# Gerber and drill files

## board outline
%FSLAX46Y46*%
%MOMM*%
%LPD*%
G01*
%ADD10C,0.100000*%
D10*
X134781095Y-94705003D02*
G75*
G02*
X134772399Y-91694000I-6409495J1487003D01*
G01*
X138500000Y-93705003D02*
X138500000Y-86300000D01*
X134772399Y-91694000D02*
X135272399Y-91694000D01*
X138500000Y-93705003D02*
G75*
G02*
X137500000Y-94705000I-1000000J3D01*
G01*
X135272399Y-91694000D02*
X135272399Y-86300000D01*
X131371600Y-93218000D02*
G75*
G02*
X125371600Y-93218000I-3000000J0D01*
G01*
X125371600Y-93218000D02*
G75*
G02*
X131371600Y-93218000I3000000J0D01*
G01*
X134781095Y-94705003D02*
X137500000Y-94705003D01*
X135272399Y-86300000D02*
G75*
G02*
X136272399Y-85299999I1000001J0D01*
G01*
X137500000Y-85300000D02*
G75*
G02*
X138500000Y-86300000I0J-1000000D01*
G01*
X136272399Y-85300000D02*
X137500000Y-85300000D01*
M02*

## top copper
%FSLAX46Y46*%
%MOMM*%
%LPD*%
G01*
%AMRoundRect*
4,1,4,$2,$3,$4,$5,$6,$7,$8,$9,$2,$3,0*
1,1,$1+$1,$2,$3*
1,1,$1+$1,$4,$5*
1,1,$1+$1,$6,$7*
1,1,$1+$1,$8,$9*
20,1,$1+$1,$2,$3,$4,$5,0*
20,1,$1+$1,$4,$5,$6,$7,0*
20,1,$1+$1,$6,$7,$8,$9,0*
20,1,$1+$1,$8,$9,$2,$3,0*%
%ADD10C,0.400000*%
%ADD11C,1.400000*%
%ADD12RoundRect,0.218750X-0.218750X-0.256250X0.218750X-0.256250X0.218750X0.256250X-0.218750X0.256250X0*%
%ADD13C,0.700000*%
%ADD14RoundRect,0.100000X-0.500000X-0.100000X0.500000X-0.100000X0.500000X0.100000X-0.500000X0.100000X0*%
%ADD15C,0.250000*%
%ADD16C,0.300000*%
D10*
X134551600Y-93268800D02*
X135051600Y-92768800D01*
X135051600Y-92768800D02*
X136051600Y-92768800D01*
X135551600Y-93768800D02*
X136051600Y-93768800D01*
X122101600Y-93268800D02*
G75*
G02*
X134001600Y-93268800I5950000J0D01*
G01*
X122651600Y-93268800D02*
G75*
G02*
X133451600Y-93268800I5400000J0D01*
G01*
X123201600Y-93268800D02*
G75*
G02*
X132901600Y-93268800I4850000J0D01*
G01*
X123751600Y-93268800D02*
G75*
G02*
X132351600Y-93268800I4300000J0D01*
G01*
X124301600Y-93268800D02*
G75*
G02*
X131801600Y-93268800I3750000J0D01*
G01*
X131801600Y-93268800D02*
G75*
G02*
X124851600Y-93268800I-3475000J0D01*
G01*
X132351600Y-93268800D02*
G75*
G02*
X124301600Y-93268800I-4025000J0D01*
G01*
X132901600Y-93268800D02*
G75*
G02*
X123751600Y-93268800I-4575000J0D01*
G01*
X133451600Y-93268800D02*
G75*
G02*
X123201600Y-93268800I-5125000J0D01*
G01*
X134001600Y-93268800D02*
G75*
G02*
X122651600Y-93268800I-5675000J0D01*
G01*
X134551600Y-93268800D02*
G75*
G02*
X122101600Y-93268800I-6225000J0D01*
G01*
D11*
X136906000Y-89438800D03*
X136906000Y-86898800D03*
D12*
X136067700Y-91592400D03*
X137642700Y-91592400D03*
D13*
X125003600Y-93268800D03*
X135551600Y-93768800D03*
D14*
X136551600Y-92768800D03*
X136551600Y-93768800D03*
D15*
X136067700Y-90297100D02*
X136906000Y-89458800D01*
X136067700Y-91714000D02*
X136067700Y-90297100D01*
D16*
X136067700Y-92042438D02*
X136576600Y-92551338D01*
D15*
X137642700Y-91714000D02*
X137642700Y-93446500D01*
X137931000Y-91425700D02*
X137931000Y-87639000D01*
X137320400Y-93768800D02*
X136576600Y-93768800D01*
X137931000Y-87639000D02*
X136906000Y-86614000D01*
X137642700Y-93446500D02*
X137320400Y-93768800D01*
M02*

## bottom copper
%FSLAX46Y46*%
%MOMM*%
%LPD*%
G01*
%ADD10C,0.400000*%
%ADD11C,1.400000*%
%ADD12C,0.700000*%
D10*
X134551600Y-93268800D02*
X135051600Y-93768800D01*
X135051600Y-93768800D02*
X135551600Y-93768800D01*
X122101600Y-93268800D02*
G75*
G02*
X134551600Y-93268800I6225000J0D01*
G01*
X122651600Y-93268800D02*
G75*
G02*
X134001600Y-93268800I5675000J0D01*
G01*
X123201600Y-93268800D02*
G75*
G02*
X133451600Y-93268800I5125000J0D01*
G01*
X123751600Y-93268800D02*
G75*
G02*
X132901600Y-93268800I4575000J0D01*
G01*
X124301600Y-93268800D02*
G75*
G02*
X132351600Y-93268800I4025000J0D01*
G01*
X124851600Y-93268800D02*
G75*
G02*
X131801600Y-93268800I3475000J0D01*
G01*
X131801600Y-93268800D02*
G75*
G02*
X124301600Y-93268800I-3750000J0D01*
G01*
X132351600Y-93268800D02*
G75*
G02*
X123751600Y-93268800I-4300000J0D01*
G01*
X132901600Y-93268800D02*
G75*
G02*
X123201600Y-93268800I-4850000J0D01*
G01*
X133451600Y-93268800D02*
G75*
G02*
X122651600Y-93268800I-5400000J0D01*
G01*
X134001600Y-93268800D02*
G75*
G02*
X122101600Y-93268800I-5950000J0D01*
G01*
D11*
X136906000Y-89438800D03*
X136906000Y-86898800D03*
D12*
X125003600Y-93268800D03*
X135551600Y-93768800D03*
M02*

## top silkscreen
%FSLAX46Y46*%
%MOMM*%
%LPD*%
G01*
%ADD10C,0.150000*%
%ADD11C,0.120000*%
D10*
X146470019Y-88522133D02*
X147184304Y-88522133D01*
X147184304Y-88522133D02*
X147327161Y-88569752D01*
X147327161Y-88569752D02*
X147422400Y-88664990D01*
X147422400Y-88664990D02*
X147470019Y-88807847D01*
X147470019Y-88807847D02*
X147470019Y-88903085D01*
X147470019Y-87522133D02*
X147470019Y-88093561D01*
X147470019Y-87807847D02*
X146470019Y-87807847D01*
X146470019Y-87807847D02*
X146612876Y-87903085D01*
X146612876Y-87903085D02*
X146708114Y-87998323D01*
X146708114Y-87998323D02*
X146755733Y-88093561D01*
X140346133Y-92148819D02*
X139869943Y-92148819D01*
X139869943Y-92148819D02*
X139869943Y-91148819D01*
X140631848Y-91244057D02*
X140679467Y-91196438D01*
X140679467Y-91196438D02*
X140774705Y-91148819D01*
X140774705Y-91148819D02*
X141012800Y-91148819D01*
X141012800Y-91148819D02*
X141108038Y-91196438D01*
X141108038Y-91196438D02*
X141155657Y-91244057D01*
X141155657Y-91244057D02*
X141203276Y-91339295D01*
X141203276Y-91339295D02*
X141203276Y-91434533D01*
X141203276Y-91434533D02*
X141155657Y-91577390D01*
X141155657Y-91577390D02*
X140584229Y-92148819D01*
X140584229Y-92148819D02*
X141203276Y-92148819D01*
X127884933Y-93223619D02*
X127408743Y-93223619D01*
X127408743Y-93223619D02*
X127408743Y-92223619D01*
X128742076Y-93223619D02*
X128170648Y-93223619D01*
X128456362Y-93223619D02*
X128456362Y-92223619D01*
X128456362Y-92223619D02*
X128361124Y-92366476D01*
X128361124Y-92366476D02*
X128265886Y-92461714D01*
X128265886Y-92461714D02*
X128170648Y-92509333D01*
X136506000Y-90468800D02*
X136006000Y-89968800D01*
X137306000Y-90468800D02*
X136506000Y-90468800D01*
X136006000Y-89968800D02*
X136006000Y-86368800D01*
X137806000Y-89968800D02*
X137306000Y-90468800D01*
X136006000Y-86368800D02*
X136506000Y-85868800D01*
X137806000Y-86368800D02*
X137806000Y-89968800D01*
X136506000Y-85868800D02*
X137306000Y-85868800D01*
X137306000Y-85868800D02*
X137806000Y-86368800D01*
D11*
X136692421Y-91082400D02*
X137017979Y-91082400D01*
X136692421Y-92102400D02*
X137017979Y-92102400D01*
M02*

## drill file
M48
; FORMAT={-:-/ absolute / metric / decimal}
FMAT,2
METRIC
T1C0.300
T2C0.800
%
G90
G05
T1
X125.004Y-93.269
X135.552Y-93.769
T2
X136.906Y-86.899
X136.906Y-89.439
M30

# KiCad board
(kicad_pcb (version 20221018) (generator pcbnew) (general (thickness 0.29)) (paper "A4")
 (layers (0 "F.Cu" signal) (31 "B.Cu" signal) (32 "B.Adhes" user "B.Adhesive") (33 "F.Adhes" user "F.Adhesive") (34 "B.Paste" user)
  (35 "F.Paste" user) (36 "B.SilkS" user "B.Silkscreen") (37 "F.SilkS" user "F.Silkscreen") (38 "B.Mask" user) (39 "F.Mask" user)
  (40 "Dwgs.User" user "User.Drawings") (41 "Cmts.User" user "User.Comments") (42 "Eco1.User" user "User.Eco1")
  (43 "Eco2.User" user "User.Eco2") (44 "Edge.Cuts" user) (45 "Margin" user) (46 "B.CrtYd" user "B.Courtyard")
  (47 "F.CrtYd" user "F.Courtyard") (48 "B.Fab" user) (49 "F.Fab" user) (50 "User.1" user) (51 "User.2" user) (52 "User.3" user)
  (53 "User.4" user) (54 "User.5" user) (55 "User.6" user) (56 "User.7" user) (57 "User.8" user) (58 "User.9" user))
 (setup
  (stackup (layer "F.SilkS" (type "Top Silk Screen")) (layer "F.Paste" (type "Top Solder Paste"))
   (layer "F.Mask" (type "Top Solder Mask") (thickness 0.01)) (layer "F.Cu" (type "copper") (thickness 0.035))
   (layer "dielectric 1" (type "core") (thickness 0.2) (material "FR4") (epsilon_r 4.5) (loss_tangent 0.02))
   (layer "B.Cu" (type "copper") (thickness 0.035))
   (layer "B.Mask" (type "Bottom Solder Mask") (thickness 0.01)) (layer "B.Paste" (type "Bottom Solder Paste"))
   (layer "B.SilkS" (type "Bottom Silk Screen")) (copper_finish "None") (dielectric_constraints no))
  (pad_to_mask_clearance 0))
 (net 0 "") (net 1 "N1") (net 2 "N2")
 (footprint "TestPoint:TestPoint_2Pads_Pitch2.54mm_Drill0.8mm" (layer "F.Cu") (at 136.906 89.4388 90)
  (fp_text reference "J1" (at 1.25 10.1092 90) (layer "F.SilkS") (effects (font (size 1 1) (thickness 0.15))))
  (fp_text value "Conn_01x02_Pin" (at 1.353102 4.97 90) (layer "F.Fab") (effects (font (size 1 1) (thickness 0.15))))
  (fp_line (start -1.03 -0.4) (end -0.53 -0.9) (stroke (width 0.15) (type solid)) (layer "F.SilkS"))
  (fp_line (start -1.03 0.4) (end -1.03 -0.4) (stroke (width 0.15) (type solid)) (layer "F.SilkS"))
  (fp_line (start -0.53 -0.9) (end 3.07 -0.9) (stroke (width 0.15) (type solid)) (layer "F.SilkS"))
  (fp_line (start -0.53 0.9) (end -1.03 0.4) (stroke (width 0.15) (type solid)) (layer "F.SilkS"))
  (fp_line (start 3.07 -0.9) (end 3.57 -0.4) (stroke (width 0.15) (type solid)) (layer "F.SilkS"))
  (fp_line (start 3.07 0.9) (end -0.53 0.9) (stroke (width 0.15) (type solid)) (layer "F.SilkS"))
  (fp_line (start 3.57 -0.4) (end 3.57 0.4) (stroke (width 0.15) (type solid)) (layer "F.SilkS"))
  (fp_line (start 3.57 0.4) (end 3.07 0.9) (stroke (width 0.15) (type solid)) (layer "F.SilkS"))
  (pad "1" thru_hole circle (at 0 0 90) (size 1.4 1.4) (drill 0.8) (layers "*.Cu" "*.Mask") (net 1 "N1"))
  (pad "2" thru_hole circle (at 2.54 0 90) (size 1.4 1.4) (drill 0.8) (layers "*.Cu" "*.Mask") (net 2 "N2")))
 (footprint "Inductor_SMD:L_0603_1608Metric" (layer "F.Cu") (at 136.8552 91.5924)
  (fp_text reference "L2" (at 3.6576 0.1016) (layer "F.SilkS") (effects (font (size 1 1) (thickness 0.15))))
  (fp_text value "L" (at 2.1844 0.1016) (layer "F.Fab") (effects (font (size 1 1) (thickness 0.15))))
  (fp_line (start -0.162779 -0.51) (end 0.162779 -0.51) (stroke (width 0.12) (type solid)) (layer "F.SilkS"))
  (fp_line (start -0.162779 0.51) (end 0.162779 0.51) (stroke (width 0.12) (type solid)) (layer "F.SilkS"))
  (pad "1" smd roundrect (at -0.7875 0) (size 0.875 0.95) (layers "F.Cu" "F.Paste" "F.Mask") (roundrect_rratio 0.25) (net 1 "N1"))
  (pad "2" smd roundrect (at 0.7875 0) (size 0.875 0.95) (layers "F.Cu" "F.Paste" "F.Mask") (roundrect_rratio 0.25) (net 2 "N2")))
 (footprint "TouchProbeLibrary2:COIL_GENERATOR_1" (layer "F.Cu") (at 128.3716 93.2688)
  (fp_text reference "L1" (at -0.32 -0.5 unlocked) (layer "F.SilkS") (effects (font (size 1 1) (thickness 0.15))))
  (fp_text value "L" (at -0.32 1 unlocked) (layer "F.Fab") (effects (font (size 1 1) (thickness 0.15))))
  (fp_line (start 6.18 0) (end 6.68 -0.5) (stroke (width 0.4) (type solid)) (layer "F.Cu"))
  (fp_line (start 6.68 -0.5) (end 7.68 -0.5) (stroke (width 0.4) (type solid)) (layer "F.Cu"))
  (fp_line (start 7.18 0.5) (end 7.68 0.5) (stroke (width 0.4) (type solid)) (layer "F.Cu"))
  (fp_arc (start -6.27 0) (mid -0.32 -5.95) (end 5.63 0) (stroke (width 0.4) (type solid)) (layer "F.Cu"))
  (fp_arc (start -5.72 0) (mid -0.32 -5.4) (end 5.08 0) (stroke (width 0.4) (type solid)) (layer "F.Cu"))
  (fp_arc (start -5.17 0) (mid -0.32 -4.85) (end 4.53 0) (stroke (width 0.4) (type solid)) (layer "F.Cu"))
  (fp_arc (start -4.62 0) (mid -0.32 -4.3) (end 3.98 0) (stroke (width 0.4) (type solid)) (layer "F.Cu"))
  (fp_arc (start -4.07 0) (mid -0.32 -3.75) (end 3.43 0) (stroke (width 0.4) (type solid)) (layer "F.Cu"))
  (fp_arc (start 3.43 0) (mid -0.045 3.475) (end -3.52 0) (stroke (width 0.4) (type solid)) (layer "F.Cu"))
  (fp_arc (start 3.98 0) (mid -0.045 4.025) (end -4.07 0) (stroke (width 0.4) (type solid)) (layer "F.Cu"))
  (fp_arc (start 4.53 0) (mid -0.045 4.575) (end -4.62 0) (stroke (width 0.4) (type solid)) (layer "F.Cu"))
  (fp_arc (start 5.08 0) (mid -0.045 5.125) (end -5.17 0) (stroke (width 0.4) (type solid)) (layer "F.Cu"))
  (fp_arc (start 5.63 0) (mid -0.045 5.675) (end -5.72 0) (stroke (width 0.4) (type solid)) (layer "F.Cu"))
  (fp_arc (start 6.18 0) (mid -0.045 6.225) (end -6.27 0) (stroke (width 0.4) (type solid)) (layer "F.Cu"))
  (fp_line (start 6.18 0) (end 6.68 0.5) (stroke (width 0.4) (type solid)) (layer "B.Cu"))
  (fp_line (start 6.68 0.5) (end 7.18 0.5) (stroke (width 0.4) (type solid)) (layer "B.Cu"))
  (fp_arc (start -6.27 0) (mid -0.045 -6.225) (end 6.18 0) (stroke (width 0.4) (type solid)) (layer "B.Cu"))
  (fp_arc (start -5.72 0) (mid -0.045 -5.675) (end 5.63 0) (stroke (width 0.4) (type solid)) (layer "B.Cu"))
  (fp_arc (start -5.17 0) (mid -0.045 -5.125) (end 5.08 0) (stroke (width 0.4) (type solid)) (layer "B.Cu"))
  (fp_arc (start -4.62 0) (mid -0.045 -4.575) (end 4.53 0) (stroke (width 0.4) (type solid)) (layer "B.Cu"))
  (fp_arc (start -4.07 0) (mid -0.045 -4.025) (end 3.98 0) (stroke (width 0.4) (type solid)) (layer "B.Cu"))
  (fp_arc (start -3.52 0) (mid -0.045 -3.475) (end 3.43 0) (stroke (width 0.4) (type solid)) (layer "B.Cu"))
  (fp_arc (start 3.43 0) (mid -0.32 3.75) (end -4.07 0) (stroke (width 0.4) (type solid)) (layer "B.Cu"))
  (fp_arc (start 3.98 0) (mid -0.32 4.3) (end -4.62 0) (stroke (width 0.4) (type solid)) (layer "B.Cu"))
  (fp_arc (start 4.53 0) (mid -0.32 4.85) (end -5.17 0) (stroke (width 0.4) (type solid)) (layer "B.Cu"))
  (fp_arc (start 5.08 0) (mid -0.32 5.4) (end -5.72 0) (stroke (width 0.4) (type solid)) (layer "B.Cu"))
  (fp_arc (start 5.63 0) (mid -0.32 5.95) (end -6.27 0) (stroke (width 0.4) (type solid)) (layer "B.Cu"))
  (pad "" thru_hole circle (at -3.368 0) (size 0.7 0.7) (drill 0.3) (layers "*.Cu" "*.Mask"))
  (pad "" thru_hole circle (at 7.18 0.5) (size 0.7 0.7) (drill 0.3) (layers "*.Cu" "*.Mask"))
  (pad "1" smd roundrect (at 8.18 -0.5) (size 1.2 0.4) (layers "F.Cu") (roundrect_rratio 0.25) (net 1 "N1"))
  (pad "2" smd roundrect (at 8.18 0.5) (size 1.2 0.4) (layers "F.Cu") (roundrect_rratio 0.25) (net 2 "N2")))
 (gr_arc (start 134.781095 94.705003) (mid 121.791901 93.237003) (end 134.772399 91.694) (stroke (width 0.1) (type default))
  (layer "Edge.Cuts"))
 (gr_line (start 138.5 93.705003) (end 138.5 86.3) (stroke (width 0.1) (type default)) (layer "Edge.Cuts"))
 (gr_line (start 134.772399 91.694) (end 135.272399 91.694) (stroke (width 0.1) (type default)) (layer "Edge.Cuts"))
 (gr_arc (start 138.5 93.705003) (mid 138.207107 94.41211) (end 137.5 94.705003) (stroke (width 0.1) (type default)) (layer "Edge.Cuts"))
 (gr_line (start 135.272399 91.694) (end 135.272399 86.3) (stroke (width 0.1) (type default)) (layer "Edge.Cuts"))
 (gr_circle (center 128.3716 93.218) (end 131.3716 93.218) (stroke (width 0.1) (type default)) (fill none) (layer "Edge.Cuts"))
 (gr_line (start 134.781095 94.705003) (end 137.5 94.705003) (stroke (width 0.1) (type default)) (layer "Edge.Cuts"))
 (gr_arc (start 135.272399 86.3) (mid 135.565292 85.592893) (end 136.272399 85.3) (stroke (width 0.1) (type default)) (layer "Edge.Cuts"))
 (gr_arc (start 137.5 85.3) (mid 138.207107 85.592893) (end 138.5 86.3) (stroke (width 0.1) (type default)) (layer "Edge.Cuts"))
 (gr_line (start 136.272399 85.3) (end 137.5 85.3) (stroke (width 0.1) (type default)) (layer "Edge.Cuts"))
 (segment (start 136.0677 90.2971) (end 136.906 89.4588) (width 0.25) (layer "F.Cu") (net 1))
 (segment (start 136.0677 91.714) (end 136.0677 90.2971) (width 0.25) (layer "F.Cu") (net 1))
 (segment (start 136.0677 92.042438) (end 136.5766 92.551338) (width 0.3) (layer "F.Cu") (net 1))
 (segment (start 137.6427 91.714) (end 137.6427 93.4465) (width 0.25) (layer "F.Cu") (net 2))
 (segment (start 137.931 91.4257) (end 137.931 87.639) (width 0.25) (layer "F.Cu") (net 2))
 (segment (start 137.3204 93.7688) (end 136.5766 93.7688) (width 0.25) (layer "F.Cu") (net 2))
 (segment (start 137.931 87.639) (end 136.906 86.614) (width 0.25) (layer "F.Cu") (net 2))
 (segment (start 137.6427 93.4465) (end 137.3204 93.7688) (width 0.25) (layer "F.Cu") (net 2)))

